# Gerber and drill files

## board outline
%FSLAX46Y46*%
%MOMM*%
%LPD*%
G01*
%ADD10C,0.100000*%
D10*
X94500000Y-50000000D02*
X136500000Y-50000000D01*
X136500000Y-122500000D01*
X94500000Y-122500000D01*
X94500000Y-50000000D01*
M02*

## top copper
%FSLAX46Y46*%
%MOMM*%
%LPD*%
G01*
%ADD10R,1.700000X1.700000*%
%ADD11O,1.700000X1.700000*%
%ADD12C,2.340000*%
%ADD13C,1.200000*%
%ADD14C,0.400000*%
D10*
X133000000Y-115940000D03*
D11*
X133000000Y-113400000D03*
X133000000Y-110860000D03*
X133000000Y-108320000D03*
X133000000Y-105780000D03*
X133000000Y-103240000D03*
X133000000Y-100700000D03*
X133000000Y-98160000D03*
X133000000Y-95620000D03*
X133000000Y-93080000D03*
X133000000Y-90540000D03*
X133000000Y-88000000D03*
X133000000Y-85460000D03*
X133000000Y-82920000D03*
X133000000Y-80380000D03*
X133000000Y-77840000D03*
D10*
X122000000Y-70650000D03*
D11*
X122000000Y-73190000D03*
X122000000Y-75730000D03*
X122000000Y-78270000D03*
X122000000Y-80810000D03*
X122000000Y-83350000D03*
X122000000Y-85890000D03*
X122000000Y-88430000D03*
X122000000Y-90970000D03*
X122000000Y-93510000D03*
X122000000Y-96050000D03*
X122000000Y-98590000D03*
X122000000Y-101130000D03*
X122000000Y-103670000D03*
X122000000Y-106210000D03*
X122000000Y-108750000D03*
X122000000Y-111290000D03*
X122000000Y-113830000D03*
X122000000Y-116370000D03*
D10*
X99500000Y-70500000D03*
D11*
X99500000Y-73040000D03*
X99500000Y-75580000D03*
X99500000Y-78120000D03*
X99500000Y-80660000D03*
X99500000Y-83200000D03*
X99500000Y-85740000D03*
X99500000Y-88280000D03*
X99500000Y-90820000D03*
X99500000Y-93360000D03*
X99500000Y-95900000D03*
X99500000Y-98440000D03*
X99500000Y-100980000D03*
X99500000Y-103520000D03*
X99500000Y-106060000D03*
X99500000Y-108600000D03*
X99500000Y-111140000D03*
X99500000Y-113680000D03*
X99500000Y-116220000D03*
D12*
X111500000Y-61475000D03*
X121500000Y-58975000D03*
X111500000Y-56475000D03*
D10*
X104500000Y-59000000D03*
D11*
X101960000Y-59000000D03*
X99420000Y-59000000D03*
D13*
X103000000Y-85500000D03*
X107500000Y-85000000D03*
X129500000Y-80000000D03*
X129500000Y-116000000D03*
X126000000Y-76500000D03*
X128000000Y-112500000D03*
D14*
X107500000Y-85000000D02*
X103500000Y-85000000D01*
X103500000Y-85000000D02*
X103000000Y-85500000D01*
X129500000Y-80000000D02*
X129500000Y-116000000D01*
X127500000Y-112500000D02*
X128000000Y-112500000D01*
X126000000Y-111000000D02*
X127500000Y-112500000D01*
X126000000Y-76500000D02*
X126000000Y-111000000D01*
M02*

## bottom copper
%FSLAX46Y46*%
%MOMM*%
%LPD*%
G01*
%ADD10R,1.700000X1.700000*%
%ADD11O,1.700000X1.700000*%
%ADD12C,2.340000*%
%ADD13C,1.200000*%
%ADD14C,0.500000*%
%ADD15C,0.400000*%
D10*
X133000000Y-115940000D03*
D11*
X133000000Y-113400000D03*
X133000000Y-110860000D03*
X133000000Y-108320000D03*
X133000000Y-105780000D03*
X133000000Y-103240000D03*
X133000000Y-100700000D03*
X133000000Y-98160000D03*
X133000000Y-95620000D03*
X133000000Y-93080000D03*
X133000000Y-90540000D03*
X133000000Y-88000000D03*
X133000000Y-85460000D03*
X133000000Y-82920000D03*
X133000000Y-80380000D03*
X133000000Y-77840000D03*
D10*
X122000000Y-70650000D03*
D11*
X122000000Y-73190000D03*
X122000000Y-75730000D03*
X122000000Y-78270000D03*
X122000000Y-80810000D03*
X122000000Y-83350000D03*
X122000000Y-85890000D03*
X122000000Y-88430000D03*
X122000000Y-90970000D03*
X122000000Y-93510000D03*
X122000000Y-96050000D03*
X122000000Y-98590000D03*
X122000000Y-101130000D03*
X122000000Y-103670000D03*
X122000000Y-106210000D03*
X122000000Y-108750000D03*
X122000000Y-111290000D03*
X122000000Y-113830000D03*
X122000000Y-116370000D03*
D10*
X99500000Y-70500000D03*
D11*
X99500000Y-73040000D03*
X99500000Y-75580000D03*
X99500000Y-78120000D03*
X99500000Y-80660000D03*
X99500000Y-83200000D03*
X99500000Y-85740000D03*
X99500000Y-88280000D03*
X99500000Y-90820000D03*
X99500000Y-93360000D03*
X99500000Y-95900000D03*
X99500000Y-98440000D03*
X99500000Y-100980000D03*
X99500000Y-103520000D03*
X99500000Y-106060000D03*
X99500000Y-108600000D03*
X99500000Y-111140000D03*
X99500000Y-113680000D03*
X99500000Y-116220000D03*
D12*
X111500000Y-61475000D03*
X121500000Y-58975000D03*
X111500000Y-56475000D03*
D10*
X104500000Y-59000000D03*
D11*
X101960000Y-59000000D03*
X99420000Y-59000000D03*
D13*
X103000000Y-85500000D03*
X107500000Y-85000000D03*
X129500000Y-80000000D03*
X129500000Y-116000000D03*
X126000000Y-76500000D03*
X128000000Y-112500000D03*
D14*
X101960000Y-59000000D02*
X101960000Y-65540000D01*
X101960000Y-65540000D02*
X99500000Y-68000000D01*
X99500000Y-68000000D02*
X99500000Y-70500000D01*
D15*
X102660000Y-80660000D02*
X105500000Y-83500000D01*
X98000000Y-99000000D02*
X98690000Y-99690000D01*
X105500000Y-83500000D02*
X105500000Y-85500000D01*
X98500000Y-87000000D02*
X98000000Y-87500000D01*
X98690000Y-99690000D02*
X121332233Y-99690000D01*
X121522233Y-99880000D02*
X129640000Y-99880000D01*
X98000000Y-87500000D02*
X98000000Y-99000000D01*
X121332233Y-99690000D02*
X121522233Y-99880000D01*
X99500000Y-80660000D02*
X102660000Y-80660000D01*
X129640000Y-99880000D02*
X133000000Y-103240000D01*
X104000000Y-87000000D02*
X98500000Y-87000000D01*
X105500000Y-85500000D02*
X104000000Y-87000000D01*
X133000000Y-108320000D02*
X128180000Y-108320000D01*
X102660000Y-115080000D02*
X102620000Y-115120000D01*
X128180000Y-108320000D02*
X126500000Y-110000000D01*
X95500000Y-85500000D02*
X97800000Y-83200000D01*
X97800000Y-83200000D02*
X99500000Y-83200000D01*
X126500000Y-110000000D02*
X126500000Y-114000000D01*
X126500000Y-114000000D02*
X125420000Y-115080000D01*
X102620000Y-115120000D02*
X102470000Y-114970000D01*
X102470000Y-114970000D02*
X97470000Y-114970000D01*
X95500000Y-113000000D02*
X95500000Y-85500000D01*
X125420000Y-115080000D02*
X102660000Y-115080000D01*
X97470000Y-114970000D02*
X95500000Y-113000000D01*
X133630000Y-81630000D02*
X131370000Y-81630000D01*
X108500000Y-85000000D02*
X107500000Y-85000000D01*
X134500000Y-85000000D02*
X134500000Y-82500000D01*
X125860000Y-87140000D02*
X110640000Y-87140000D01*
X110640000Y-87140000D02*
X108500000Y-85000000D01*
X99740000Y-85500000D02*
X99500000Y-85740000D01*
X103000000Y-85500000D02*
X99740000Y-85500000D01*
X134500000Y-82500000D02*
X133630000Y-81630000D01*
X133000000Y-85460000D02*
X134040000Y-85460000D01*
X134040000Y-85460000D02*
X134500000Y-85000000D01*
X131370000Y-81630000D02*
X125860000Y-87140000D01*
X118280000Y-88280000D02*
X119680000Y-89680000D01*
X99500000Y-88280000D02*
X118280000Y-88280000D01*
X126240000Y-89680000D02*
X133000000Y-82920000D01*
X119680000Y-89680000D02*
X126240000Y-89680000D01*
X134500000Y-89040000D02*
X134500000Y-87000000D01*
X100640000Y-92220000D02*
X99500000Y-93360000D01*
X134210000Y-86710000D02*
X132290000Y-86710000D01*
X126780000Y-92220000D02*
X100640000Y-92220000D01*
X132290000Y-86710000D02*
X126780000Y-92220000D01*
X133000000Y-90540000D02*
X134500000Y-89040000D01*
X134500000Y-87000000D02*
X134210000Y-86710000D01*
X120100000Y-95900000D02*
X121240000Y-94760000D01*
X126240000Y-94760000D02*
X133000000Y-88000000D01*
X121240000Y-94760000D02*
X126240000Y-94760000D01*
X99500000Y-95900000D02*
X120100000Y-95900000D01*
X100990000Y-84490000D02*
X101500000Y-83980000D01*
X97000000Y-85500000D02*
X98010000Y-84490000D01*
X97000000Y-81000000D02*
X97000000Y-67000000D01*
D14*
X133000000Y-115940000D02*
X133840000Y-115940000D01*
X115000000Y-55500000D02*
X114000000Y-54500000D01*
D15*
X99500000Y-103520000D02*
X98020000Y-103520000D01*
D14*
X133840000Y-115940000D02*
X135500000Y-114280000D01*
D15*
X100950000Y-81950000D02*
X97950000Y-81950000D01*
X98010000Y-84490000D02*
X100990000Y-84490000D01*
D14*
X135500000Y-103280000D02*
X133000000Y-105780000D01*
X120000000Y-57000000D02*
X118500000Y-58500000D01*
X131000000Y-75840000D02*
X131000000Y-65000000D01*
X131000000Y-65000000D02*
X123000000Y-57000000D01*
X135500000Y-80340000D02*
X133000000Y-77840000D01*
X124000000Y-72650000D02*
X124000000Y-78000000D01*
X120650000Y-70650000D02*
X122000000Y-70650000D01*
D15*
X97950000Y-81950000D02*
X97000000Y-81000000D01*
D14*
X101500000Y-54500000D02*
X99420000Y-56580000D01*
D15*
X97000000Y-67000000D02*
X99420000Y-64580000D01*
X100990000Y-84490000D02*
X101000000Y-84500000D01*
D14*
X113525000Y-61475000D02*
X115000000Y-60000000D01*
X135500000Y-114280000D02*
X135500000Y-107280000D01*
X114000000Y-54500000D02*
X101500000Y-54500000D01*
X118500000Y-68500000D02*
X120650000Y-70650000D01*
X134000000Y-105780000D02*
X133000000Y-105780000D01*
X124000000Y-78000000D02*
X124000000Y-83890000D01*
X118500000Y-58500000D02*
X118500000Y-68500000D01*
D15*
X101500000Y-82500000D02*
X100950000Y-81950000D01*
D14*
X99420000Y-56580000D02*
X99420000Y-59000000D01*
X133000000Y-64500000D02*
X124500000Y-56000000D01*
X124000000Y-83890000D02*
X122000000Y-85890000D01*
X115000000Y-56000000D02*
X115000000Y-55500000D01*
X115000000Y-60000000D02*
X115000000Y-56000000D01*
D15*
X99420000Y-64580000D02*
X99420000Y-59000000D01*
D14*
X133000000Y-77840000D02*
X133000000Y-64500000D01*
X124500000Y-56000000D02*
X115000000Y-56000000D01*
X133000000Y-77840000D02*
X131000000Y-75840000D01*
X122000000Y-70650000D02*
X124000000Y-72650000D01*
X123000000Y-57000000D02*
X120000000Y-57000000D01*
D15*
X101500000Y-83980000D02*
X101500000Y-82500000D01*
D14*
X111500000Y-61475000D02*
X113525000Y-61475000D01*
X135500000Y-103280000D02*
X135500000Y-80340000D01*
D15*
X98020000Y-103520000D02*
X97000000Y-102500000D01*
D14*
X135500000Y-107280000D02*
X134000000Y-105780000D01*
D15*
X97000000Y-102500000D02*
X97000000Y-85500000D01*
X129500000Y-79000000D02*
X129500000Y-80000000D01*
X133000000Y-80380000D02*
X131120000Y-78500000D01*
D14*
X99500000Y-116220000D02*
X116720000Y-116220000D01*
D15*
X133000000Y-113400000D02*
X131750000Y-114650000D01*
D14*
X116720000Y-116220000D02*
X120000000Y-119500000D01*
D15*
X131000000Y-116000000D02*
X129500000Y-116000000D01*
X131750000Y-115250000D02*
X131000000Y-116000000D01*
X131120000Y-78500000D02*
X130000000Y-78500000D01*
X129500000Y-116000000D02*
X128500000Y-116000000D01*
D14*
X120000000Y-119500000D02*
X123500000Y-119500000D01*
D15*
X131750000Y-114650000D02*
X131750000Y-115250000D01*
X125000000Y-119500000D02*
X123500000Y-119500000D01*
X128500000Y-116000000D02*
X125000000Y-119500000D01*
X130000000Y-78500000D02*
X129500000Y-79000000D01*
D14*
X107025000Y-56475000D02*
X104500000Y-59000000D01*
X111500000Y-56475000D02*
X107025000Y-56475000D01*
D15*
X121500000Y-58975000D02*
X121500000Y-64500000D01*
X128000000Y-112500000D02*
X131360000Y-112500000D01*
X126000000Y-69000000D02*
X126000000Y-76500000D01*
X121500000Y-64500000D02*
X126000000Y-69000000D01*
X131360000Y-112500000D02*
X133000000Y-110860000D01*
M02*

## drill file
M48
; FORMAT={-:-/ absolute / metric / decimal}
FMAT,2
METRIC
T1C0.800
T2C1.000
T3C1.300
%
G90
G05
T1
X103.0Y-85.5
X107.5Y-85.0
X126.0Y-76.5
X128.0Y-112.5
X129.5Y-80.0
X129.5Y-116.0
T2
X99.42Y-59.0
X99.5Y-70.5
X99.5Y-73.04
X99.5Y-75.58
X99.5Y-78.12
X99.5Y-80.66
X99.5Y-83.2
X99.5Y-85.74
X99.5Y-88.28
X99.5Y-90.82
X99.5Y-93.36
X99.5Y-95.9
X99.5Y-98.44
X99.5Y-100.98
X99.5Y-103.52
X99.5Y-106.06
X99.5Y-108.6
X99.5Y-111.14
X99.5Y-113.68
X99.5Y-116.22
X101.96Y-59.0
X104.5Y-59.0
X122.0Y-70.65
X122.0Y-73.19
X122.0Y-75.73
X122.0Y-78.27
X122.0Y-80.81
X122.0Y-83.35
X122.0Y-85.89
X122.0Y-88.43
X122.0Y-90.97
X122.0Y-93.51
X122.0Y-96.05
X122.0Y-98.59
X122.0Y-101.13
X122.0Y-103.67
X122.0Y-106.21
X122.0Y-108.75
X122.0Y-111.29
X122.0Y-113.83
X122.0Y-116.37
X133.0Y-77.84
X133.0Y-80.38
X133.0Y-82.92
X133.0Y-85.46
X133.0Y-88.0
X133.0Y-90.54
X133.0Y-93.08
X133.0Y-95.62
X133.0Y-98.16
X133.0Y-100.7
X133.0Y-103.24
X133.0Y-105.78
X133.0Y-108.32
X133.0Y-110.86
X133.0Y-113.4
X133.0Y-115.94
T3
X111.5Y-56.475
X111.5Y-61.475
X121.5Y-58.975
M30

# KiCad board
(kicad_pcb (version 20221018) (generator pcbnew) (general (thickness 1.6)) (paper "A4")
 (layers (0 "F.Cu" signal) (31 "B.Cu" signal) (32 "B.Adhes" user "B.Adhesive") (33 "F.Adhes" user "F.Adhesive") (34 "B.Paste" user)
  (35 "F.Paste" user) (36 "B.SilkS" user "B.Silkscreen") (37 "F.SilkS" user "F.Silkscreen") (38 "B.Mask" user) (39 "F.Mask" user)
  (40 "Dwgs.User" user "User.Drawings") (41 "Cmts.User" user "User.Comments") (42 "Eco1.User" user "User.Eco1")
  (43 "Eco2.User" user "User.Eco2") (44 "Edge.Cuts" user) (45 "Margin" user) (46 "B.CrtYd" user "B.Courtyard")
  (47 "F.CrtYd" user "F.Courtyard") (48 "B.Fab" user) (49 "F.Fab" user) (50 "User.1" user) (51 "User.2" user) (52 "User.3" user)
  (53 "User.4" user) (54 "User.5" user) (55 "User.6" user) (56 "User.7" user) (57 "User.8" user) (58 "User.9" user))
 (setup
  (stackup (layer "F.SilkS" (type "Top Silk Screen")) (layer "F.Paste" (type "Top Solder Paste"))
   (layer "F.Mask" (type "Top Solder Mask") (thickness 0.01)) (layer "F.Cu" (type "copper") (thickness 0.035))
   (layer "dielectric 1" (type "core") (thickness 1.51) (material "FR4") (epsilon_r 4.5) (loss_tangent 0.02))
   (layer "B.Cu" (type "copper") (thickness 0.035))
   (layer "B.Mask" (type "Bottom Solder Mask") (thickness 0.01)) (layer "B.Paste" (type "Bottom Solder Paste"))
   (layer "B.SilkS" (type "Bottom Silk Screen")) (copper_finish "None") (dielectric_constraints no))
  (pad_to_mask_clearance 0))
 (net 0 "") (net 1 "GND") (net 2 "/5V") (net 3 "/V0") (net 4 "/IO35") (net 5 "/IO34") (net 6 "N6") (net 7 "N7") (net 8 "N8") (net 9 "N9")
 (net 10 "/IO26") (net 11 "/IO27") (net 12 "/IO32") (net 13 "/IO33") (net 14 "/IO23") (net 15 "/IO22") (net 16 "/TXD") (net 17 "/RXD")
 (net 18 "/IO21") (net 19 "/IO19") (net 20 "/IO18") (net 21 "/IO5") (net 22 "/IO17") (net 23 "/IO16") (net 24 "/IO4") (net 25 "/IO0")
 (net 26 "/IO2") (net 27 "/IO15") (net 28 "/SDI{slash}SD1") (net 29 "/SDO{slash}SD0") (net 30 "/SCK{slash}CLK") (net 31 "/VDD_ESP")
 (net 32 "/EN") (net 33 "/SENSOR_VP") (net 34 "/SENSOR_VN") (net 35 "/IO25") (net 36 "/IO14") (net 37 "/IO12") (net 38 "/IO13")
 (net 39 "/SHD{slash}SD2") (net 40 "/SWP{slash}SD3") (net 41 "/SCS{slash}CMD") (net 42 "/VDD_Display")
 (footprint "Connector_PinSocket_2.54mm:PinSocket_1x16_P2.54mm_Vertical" (layer "F.Cu") (at 133 115.94 180)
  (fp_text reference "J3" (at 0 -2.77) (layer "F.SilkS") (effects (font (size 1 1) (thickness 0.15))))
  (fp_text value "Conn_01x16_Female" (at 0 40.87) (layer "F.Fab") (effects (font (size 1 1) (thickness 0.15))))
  (pad "1" thru_hole rect (at 0 0 180) (size 1.7 1.7) (drill 1) (layers "*.Cu" "*.Mask") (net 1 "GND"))
  (pad "2" thru_hole oval (at 0 2.54 180) (size 1.7 1.7) (drill 1) (layers "*.Cu" "*.Mask") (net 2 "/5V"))
  (pad "3" thru_hole oval (at 0 5.08 180) (size 1.7 1.7) (drill 1) (layers "*.Cu" "*.Mask") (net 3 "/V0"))
  (pad "4" thru_hole oval (at 0 7.62 180) (size 1.7 1.7) (drill 1) (layers "*.Cu" "*.Mask") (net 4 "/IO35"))
  (pad "5" thru_hole oval (at 0 10.16 180) (size 1.7 1.7) (drill 1) (layers "*.Cu" "*.Mask") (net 1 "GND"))
  (pad "6" thru_hole oval (at 0 12.7 180) (size 1.7 1.7) (drill 1) (layers "*.Cu" "*.Mask") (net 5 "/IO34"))
  (pad "7" thru_hole oval (at 0 15.24 180) (size 1.7 1.7) (drill 1) (layers "*.Cu" "*.Mask") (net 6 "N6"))
  (pad "8" thru_hole oval (at 0 17.78 180) (size 1.7 1.7) (drill 1) (layers "*.Cu" "*.Mask") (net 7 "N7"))
  (pad "9" thru_hole oval (at 0 20.32 180) (size 1.7 1.7) (drill 1) (layers "*.Cu" "*.Mask") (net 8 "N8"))
  (pad "10" thru_hole oval (at 0 22.86 180) (size 1.7 1.7) (drill 1) (layers "*.Cu" "*.Mask") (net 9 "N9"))
  (pad "11" thru_hole oval (at 0 25.4 180) (size 1.7 1.7) (drill 1) (layers "*.Cu" "*.Mask") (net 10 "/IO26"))
  (pad "12" thru_hole oval (at 0 27.94 180) (size 1.7 1.7) (drill 1) (layers "*.Cu" "*.Mask") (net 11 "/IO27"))
  (pad "13" thru_hole oval (at 0 30.48 180) (size 1.7 1.7) (drill 1) (layers "*.Cu" "*.Mask") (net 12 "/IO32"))
  (pad "14" thru_hole oval (at 0 33.02 180) (size 1.7 1.7) (drill 1) (layers "*.Cu" "*.Mask") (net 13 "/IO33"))
  (pad "15" thru_hole oval (at 0 35.56 180) (size 1.7 1.7) (drill 1) (layers "*.Cu" "*.Mask") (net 2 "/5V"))
  (pad "16" thru_hole oval (at 0 38.1 180) (size 1.7 1.7) (drill 1) (layers "*.Cu" "*.Mask") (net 1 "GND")))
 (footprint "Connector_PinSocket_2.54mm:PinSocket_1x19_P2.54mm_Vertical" (layer "F.Cu") (at 122 70.65)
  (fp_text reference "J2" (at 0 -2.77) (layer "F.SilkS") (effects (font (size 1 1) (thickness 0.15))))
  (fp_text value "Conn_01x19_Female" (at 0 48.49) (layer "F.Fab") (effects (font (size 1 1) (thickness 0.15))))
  (pad "1" thru_hole rect (at 0 0) (size 1.7 1.7) (drill 1) (layers "*.Cu" "*.Mask") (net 1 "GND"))
  (pad "2" thru_hole oval (at 0 2.54) (size 1.7 1.7) (drill 1) (layers "*.Cu" "*.Mask") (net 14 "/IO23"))
  (pad "3" thru_hole oval (at 0 5.08) (size 1.7 1.7) (drill 1) (layers "*.Cu" "*.Mask") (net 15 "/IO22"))
  (pad "4" thru_hole oval (at 0 7.62) (size 1.7 1.7) (drill 1) (layers "*.Cu" "*.Mask") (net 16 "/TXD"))
  (pad "5" thru_hole oval (at 0 10.16) (size 1.7 1.7) (drill 1) (layers "*.Cu" "*.Mask") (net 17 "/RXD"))
  (pad "6" thru_hole oval (at 0 12.7) (size 1.7 1.7) (drill 1) (layers "*.Cu" "*.Mask") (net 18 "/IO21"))
  (pad "7" thru_hole oval (at 0 15.24) (size 1.7 1.7) (drill 1) (layers "*.Cu" "*.Mask") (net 1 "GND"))
  (pad "8" thru_hole oval (at 0 17.78) (size 1.7 1.7) (drill 1) (layers "*.Cu" "*.Mask") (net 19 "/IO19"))
  (pad "9" thru_hole oval (at 0 20.32) (size 1.7 1.7) (drill 1) (layers "*.Cu" "*.Mask") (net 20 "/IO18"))
  (pad "10" thru_hole oval (at 0 22.86) (size 1.7 1.7) (drill 1) (layers "*.Cu" "*.Mask") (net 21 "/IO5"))
  (pad "11" thru_hole oval (at 0 25.4) (size 1.7 1.7) (drill 1) (layers "*.Cu" "*.Mask") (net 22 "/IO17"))
  (pad "12" thru_hole oval (at 0 27.94) (size 1.7 1.7) (drill 1) (layers "*.Cu" "*.Mask") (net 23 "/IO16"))
  (pad "13" thru_hole oval (at 0 30.48) (size 1.7 1.7) (drill 1) (layers "*.Cu" "*.Mask") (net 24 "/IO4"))
  (pad "14" thru_hole oval (at 0 33.02) (size 1.7 1.7) (drill 1) (layers "*.Cu" "*.Mask") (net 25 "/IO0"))
  (pad "15" thru_hole oval (at 0 35.56) (size 1.7 1.7) (drill 1) (layers "*.Cu" "*.Mask") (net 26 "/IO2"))
  (pad "16" thru_hole oval (at 0 38.1) (size 1.7 1.7) (drill 1) (layers "*.Cu" "*.Mask") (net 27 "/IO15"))
  (pad "17" thru_hole oval (at 0 40.64) (size 1.7 1.7) (drill 1) (layers "*.Cu" "*.Mask") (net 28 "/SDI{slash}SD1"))
  (pad "18" thru_hole oval (at 0 43.18) (size 1.7 1.7) (drill 1) (layers "*.Cu" "*.Mask") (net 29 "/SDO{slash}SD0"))
  (pad "19" thru_hole oval (at 0 45.72) (size 1.7 1.7) (drill 1) (layers "*.Cu" "*.Mask") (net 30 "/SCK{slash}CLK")))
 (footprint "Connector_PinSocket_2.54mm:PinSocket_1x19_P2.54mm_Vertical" (layer "F.Cu") (at 99.5 70.5)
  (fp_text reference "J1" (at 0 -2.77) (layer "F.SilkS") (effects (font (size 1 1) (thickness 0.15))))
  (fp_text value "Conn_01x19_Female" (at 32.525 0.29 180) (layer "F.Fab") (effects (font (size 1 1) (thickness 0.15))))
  (pad "1" thru_hole rect (at 0 0) (size 1.7 1.7) (drill 1) (layers "*.Cu" "*.Mask") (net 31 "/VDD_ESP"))
  (pad "2" thru_hole oval (at 0 2.54) (size 1.7 1.7) (drill 1) (layers "*.Cu" "*.Mask") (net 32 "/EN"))
  (pad "3" thru_hole oval (at 0 5.08) (size 1.7 1.7) (drill 1) (layers "*.Cu" "*.Mask") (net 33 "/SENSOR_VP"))
  (pad "4" thru_hole oval (at 0 7.62) (size 1.7 1.7) (drill 1) (layers "*.Cu" "*.Mask") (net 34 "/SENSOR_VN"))
  (pad "5" thru_hole oval (at 0 10.16) (size 1.7 1.7) (drill 1) (layers "*.Cu" "*.Mask") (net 5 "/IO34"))
  (pad "6" thru_hole oval (at 0 12.7) (size 1.7 1.7) (drill 1) (layers "*.Cu" "*.Mask") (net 4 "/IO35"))
  (pad "7" thru_hole oval (at 0 15.24) (size 1.7 1.7) (drill 1) (layers "*.Cu" "*.Mask") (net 12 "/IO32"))
  (pad "8" thru_hole oval (at 0 17.78) (size 1.7 1.7) (drill 1) (layers "*.Cu" "*.Mask") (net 13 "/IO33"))
  (pad "9" thru_hole oval (at 0 20.32) (size 1.7 1.7) (drill 1) (layers "*.Cu" "*.Mask") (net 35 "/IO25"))
  (pad "10" thru_hole oval (at 0 22.86) (size 1.7 1.7) (drill 1) (layers "*.Cu" "*.Mask") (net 10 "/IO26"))
  (pad "11" thru_hole oval (at 0 25.4) (size 1.7 1.7) (drill 1) (layers "*.Cu" "*.Mask") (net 11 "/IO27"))
  (pad "12" thru_hole oval (at 0 27.94) (size 1.7 1.7) (drill 1) (layers "*.Cu" "*.Mask") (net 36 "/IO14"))
  (pad "13" thru_hole oval (at 0 30.48) (size 1.7 1.7) (drill 1) (layers "*.Cu" "*.Mask") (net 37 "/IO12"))
  (pad "14" thru_hole oval (at 0 33.02) (size 1.7 1.7) (drill 1) (layers "*.Cu" "*.Mask") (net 1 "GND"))
  (pad "15" thru_hole oval (at 0 35.56) (size 1.7 1.7) (drill 1) (layers "*.Cu" "*.Mask") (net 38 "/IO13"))
  (pad "16" thru_hole oval (at 0 38.1) (size 1.7 1.7) (drill 1) (layers "*.Cu" "*.Mask") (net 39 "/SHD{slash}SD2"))
  (pad "17" thru_hole oval (at 0 40.64) (size 1.7 1.7) (drill 1) (layers "*.Cu" "*.Mask") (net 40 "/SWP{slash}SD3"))
  (pad "18" thru_hole oval (at 0 43.18) (size 1.7 1.7) (drill 1) (layers "*.Cu" "*.Mask") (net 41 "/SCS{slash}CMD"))
  (pad "19" thru_hole oval (at 0 45.72) (size 1.7 1.7) (drill 1) (layers "*.Cu" "*.Mask") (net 2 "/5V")))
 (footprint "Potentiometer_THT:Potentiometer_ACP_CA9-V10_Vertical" (layer "F.Cu") (at 111.5 61.475)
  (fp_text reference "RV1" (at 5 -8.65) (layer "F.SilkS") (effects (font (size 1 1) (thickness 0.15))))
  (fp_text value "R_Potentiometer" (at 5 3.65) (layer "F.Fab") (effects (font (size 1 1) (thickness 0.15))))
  (pad "1" thru_hole circle (at 0 0) (size 2.34 2.34) (drill 1.3) (layers "*.Cu" "*.Mask") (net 1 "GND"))
  (pad "2" thru_hole circle (at 10 -2.5) (size 2.34 2.34) (drill 1.3) (layers "*.Cu" "*.Mask") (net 3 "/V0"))
  (pad "3" thru_hole circle (at 0 -5) (size 2.34 2.34) (drill 1.3) (layers "*.Cu" "*.Mask") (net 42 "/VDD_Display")))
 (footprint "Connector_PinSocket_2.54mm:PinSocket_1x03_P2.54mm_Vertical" (layer "F.Cu") (at 104.5 59 -90)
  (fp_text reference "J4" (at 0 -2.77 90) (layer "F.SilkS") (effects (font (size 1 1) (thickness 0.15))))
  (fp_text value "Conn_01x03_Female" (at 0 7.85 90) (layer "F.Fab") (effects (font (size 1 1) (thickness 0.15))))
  (pad "1" thru_hole rect (at 0 0 270) (size 1.7 1.7) (drill 1) (layers "*.Cu" "*.Mask") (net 42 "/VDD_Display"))
  (pad "2" thru_hole oval (at 0 2.54 270) (size 1.7 1.7) (drill 1) (layers "*.Cu" "*.Mask") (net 31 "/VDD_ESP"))
  (pad "3" thru_hole oval (at 0 5.08 270) (size 1.7 1.7) (drill 1) (layers "*.Cu" "*.Mask") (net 1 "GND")))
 (gr_rect (start 94.5 50) (end 136.5 122.5) (stroke (width 0.1) (type solid)) (fill none) (layer "Edge.Cuts"))
 (segment (start 101.96 59) (end 101.96 65.54) (width 0.5) (layer "B.Cu") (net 31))
 (segment (start 101.96 65.54) (end 99.5 68) (width 0.5) (layer "B.Cu") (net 31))
 (segment (start 99.5 68) (end 99.5 70.5) (width 0.5) (layer "B.Cu") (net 31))
 (segment (start 102.66 80.66) (end 105.5 83.5) (width 0.4) (layer "B.Cu") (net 5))
 (segment (start 98 99) (end 98.69 99.69) (width 0.4) (layer "B.Cu") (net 5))
 (segment (start 105.5 83.5) (end 105.5 85.5) (width 0.4) (layer "B.Cu") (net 5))
 (segment (start 98.5 87) (end 98 87.5) (width 0.4) (layer "B.Cu") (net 5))
 (segment (start 98.69 99.69) (end 121.332233 99.69) (width 0.4) (layer "B.Cu") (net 5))
 (segment (start 121.522233 99.88) (end 129.64 99.88) (width 0.4) (layer "B.Cu") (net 5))
 (segment (start 98 87.5) (end 98 99) (width 0.4) (layer "B.Cu") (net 5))
 (segment (start 121.332233 99.69) (end 121.522233 99.88) (width 0.4) (layer "B.Cu") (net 5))
 (segment (start 99.5 80.66) (end 102.66 80.66) (width 0.4) (layer "B.Cu") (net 5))
 (segment (start 129.64 99.88) (end 133 103.24) (width 0.4) (layer "B.Cu") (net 5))
 (segment (start 104 87) (end 98.5 87) (width 0.4) (layer "B.Cu") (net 5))
 (segment (start 105.5 85.5) (end 104 87) (width 0.4) (layer "B.Cu") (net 5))
 (segment (start 133 108.32) (end 128.18 108.32) (width 0.4) (layer "B.Cu") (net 4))
 (segment (start 102.66 115.08) (end 102.62 115.12) (width 0.4) (layer "B.Cu") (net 4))
 (segment (start 128.18 108.32) (end 126.5 110) (width 0.4) (layer "B.Cu") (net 4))
 (segment (start 95.5 85.5) (end 97.8 83.2) (width 0.4) (layer "B.Cu") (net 4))
 (segment (start 97.8 83.2) (end 99.5 83.2) (width 0.4) (layer "B.Cu") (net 4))
 (segment (start 126.5 110) (end 126.5 114) (width 0.4) (layer "B.Cu") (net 4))
 (segment (start 126.5 114) (end 125.42 115.08) (width 0.4) (layer "B.Cu") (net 4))
 (segment (start 102.62 115.12) (end 102.47 114.97) (width 0.4) (layer "B.Cu") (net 4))
 (segment (start 102.47 114.97) (end 97.47 114.97) (width 0.4) (layer "B.Cu") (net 4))
 (segment (start 95.5 113) (end 95.5 85.5) (width 0.4) (layer "B.Cu") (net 4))
 (segment (start 125.42 115.08) (end 102.66 115.08) (width 0.4) (layer "B.Cu") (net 4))
 (segment (start 97.47 114.97) (end 95.5 113) (width 0.4) (layer "B.Cu") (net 4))
 (segment (start 107.5 85) (end 103.5 85) (width 0.4) (layer "F.Cu") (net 12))
 (segment (start 103.5 85) (end 103 85.5) (width 0.4) (layer "F.Cu") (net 12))
 (via (at 103 85.5) (size 1.2) (drill 0.8) (layers "F.Cu" "B.Cu") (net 12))
 (via (at 107.5 85) (size 1.2) (drill 0.8) (layers "F.Cu" "B.Cu") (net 12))
 (segment (start 133.63 81.63) (end 131.37 81.63) (width 0.4) (layer "B.Cu") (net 12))
 (segment (start 108.5 85) (end 107.5 85) (width 0.4) (layer "B.Cu") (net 12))
 (segment (start 134.5 85) (end 134.5 82.5) (width 0.4) (layer "B.Cu") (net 12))
 (segment (start 125.86 87.14) (end 110.64 87.14) (width 0.4) (layer "B.Cu") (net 12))
 (segment (start 110.64 87.14) (end 108.5 85) (width 0.4) (layer "B.Cu") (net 12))
 (segment (start 99.74 85.5) (end 99.5 85.74) (width 0.4) (layer "B.Cu") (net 12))
 (segment (start 103 85.5) (end 99.74 85.5) (width 0.4) (layer "B.Cu") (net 12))
 (segment (start 134.5 82.5) (end 133.63 81.63) (width 0.4) (layer "B.Cu") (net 12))
 (segment (start 133 85.46) (end 134.04 85.46) (width 0.4) (layer "B.Cu") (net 12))
 (segment (start 134.04 85.46) (end 134.5 85) (width 0.4) (layer "B.Cu") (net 12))
 (segment (start 131.37 81.63) (end 125.86 87.14) (width 0.4) (layer "B.Cu") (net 12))
 (segment (start 118.28 88.28) (end 119.68 89.68) (width 0.4) (layer "B.Cu") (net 13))
 (segment (start 99.5 88.28) (end 118.28 88.28) (width 0.4) (layer "B.Cu") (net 13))
 (segment (start 126.24 89.68) (end 133 82.92) (width 0.4) (layer "B.Cu") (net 13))
 (segment (start 119.68 89.68) (end 126.24 89.68) (width 0.4) (layer "B.Cu") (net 13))
 (segment (start 134.5 89.04) (end 134.5 87) (width 0.4) (layer "B.Cu") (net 10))
 (segment (start 100.64 92.22) (end 99.5 93.36) (width 0.4) (layer "B.Cu") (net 10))
 (segment (start 134.21 86.71) (end 132.29 86.71) (width 0.4) (layer "B.Cu") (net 10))
 (segment (start 126.78 92.22) (end 100.64 92.22) (width 0.4) (layer "B.Cu") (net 10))
 (segment (start 132.29 86.71) (end 126.78 92.22) (width 0.4) (layer "B.Cu") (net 10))
 (segment (start 133 90.54) (end 134.5 89.04) (width 0.4) (layer "B.Cu") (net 10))
 (segment (start 134.5 87) (end 134.21 86.71) (width 0.4) (layer "B.Cu") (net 10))
 (segment (start 120.1 95.9) (end 121.24 94.76) (width 0.4) (layer "B.Cu") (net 11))
 (segment (start 126.24 94.76) (end 133 88) (width 0.4) (layer "B.Cu") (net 11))
 (segment (start 121.24 94.76) (end 126.24 94.76) (width 0.4) (layer "B.Cu") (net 11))
 (segment (start 99.5 95.9) (end 120.1 95.9) (width 0.4) (layer "B.Cu") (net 11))
 (segment (start 100.99 84.49) (end 101.5 83.98) (width 0.4) (layer "B.Cu") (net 1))
 (segment (start 97 85.5) (end 98.01 84.49) (width 0.4) (layer "B.Cu") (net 1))
 (segment (start 97 81) (end 97 67) (width 0.4) (layer "B.Cu") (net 1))
 (segment (start 133 115.94) (end 133.84 115.94) (width 0.5) (layer "B.Cu") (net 1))
 (segment (start 115 55.5) (end 114 54.5) (width 0.5) (layer "B.Cu") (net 1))
 (segment (start 99.5 103.52) (end 98.02 103.52) (width 0.4) (layer "B.Cu") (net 1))
 (segment (start 133.84 115.94) (end 135.5 114.28) (width 0.5) (layer "B.Cu") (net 1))
 (segment (start 100.95 81.95) (end 97.95 81.95) (width 0.4) (layer "B.Cu") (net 1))
 (segment (start 98.01 84.49) (end 100.99 84.49) (width 0.4) (layer "B.Cu") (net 1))
 (segment (start 135.5 103.28) (end 133 105.78) (width 0.5) (layer "B.Cu") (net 1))
 (segment (start 120 57) (end 118.5 58.5) (width 0.5) (layer "B.Cu") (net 1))
 (segment (start 131 75.84) (end 131 65) (width 0.5) (layer "B.Cu") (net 1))
 (segment (start 131 65) (end 123 57) (width 0.5) (layer "B.Cu") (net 1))
 (segment (start 135.5 80.34) (end 133 77.84) (width 0.5) (layer "B.Cu") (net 1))
 (segment (start 124 72.65) (end 124 78) (width 0.5) (layer "B.Cu") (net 1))
 (segment (start 120.65 70.65) (end 122 70.65) (width 0.5) (layer "B.Cu") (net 1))
 (segment (start 97.95 81.95) (end 97 81) (width 0.4) (layer "B.Cu") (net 1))
 (segment (start 101.5 54.5) (end 99.42 56.58) (width 0.5) (layer "B.Cu") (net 1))
 (segment (start 97 67) (end 99.42 64.58) (width 0.4) (layer "B.Cu") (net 1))
 (segment (start 100.99 84.49) (end 101 84.5) (width 0.4) (layer "B.Cu") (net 1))
 (segment (start 113.525 61.475) (end 115 60) (width 0.5) (layer "B.Cu") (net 1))
 (segment (start 135.5 114.28) (end 135.5 107.28) (width 0.5) (layer "B.Cu") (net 1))
 (segment (start 114 54.5) (end 101.5 54.5) (width 0.5) (layer "B.Cu") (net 1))
 (segment (start 118.5 68.5) (end 120.65 70.65) (width 0.5) (layer "B.Cu") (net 1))
 (segment (start 134 105.78) (end 133 105.78) (width 0.5) (layer "B.Cu") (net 1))
 (segment (start 124 78) (end 124 83.89) (width 0.5) (layer "B.Cu") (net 1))
 (segment (start 118.5 58.5) (end 118.5 68.5) (width 0.5) (layer "B.Cu") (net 1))
 (segment (start 101.5 82.5) (end 100.95 81.95) (width 0.4) (layer "B.Cu") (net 1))
 (segment (start 99.42 56.58) (end 99.42 59) (width 0.5) (layer "B.Cu") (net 1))
 (segment (start 133 64.5) (end 124.5 56) (width 0.5) (layer "B.Cu") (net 1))
 (segment (start 124 83.89) (end 122 85.89) (width 0.5) (layer "B.Cu") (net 1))
 (segment (start 115 56) (end 115 55.5) (width 0.5) (layer "B.Cu") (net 1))
 (segment (start 115 60) (end 115 56) (width 0.5) (layer "B.Cu") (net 1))
 (segment (start 99.42 64.58) (end 99.42 59) (width 0.4) (layer "B.Cu") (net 1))
 (segment (start 133 77.84) (end 133 64.5) (width 0.5) (layer "B.Cu") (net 1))
 (segment (start 124.5 56) (end 115 56) (width 0.5) (layer "B.Cu") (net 1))
 (segment (start 133 77.84) (end 131 75.84) (width 0.5) (layer "B.Cu") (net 1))
 (segment (start 122 70.65) (end 124 72.65) (width 0.5) (layer "B.Cu") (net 1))
 (segment (start 123 57) (end 120 57) (width 0.5) (layer "B.Cu") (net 1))
 (segment (start 101.5 83.98) (end 101.5 82.5) (width 0.4) (layer "B.Cu") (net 1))
 (segment (start 111.5 61.475) (end 113.525 61.475) (width 0.5) (layer "B.Cu") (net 1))
 (segment (start 135.5 103.28) (end 135.5 80.34) (width 0.5) (layer "B.Cu") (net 1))
 (segment (start 98.02 103.52) (end 97 102.5) (width 0.4) (layer "B.Cu") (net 1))
 (segment (start 135.5 107.28) (end 134 105.78) (width 0.5) (layer "B.Cu") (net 1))
 (segment (start 97 102.5) (end 97 85.5) (width 0.4) (layer "B.Cu") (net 1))
 (segment (start 129.5 80) (end 129.5 116) (width 0.4) (layer "F.Cu") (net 2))
 (via (at 129.5 80) (size 1.2) (drill 0.8) (layers "F.Cu" "B.Cu") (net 2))
 (via (at 129.5 116) (size 1.2) (drill 0.8) (layers "F.Cu" "B.Cu") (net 2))
 (segment (start 129.5 79) (end 129.5 80) (width 0.4) (layer "B.Cu") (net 2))
 (segment (start 133 80.38) (end 131.12 78.5) (width 0.4) (layer "B.Cu") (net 2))
 (segment (start 99.5 116.22) (end 116.72 116.22) (width 0.5) (layer "B.Cu") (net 2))
 (segment (start 133 113.4) (end 131.75 114.65) (width 0.4) (layer "B.Cu") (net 2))
 (segment (start 116.72 116.22) (end 120 119.5) (width 0.5) (layer "B.Cu") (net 2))
 (segment (start 131 116) (end 129.5 116) (width 0.4) (layer "B.Cu") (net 2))
 (segment (start 131.75 115.25) (end 131 116) (width 0.4) (layer "B.Cu") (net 2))
 (segment (start 131.12 78.5) (end 130 78.5) (width 0.4) (layer "B.Cu") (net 2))
 (segment (start 129.5 116) (end 128.5 116) (width 0.4) (layer "B.Cu") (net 2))
 (segment (start 120 119.5) (end 123.5 119.5) (width 0.5) (layer "B.Cu") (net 2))
 (segment (start 131.75 114.65) (end 131.75 115.25) (width 0.4) (layer "B.Cu") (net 2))
 (segment (start 125 119.5) (end 123.5 119.5) (width 0.4) (layer "B.Cu") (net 2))
 (segment (start 128.5 116) (end 125 119.5) (width 0.4) (layer "B.Cu") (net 2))
 (segment (start 130 78.5) (end 129.5 79) (width 0.4) (layer "B.Cu") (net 2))
 (segment (start 107.025 56.475) (end 104.5 59) (width 0.5) (layer "B.Cu") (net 42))
 (segment (start 111.5 56.475) (end 107.025 56.475) (width 0.5) (layer "B.Cu") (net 42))
 (segment (start 127.5 112.5) (end 128 112.5) (width 0.4) (layer "F.Cu") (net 3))
 (segment (start 126 111) (end 127.5 112.5) (width 0.4) (layer "F.Cu") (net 3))
 (segment (start 126 76.5) (end 126 111) (width 0.4) (layer "F.Cu") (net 3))
 (via (at 126 76.5) (size 1.2) (drill 0.8) (layers "F.Cu" "B.Cu") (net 3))
 (via (at 128 112.5) (size 1.2) (drill 0.8) (layers "F.Cu" "B.Cu") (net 3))
 (segment (start 121.5 58.975) (end 121.5 64.5) (width 0.4) (layer "B.Cu") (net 3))
 (segment (start 128 112.5) (end 131.36 112.5) (width 0.4) (layer "B.Cu") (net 3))
 (segment (start 126 69) (end 126 76.5) (width 0.4) (layer "B.Cu") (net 3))
 (segment (start 121.5 64.5) (end 126 69) (width 0.4) (layer "B.Cu") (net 3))
 (segment (start 131.36 112.5) (end 133 110.86) (width 0.4) (layer "B.Cu") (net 3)))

